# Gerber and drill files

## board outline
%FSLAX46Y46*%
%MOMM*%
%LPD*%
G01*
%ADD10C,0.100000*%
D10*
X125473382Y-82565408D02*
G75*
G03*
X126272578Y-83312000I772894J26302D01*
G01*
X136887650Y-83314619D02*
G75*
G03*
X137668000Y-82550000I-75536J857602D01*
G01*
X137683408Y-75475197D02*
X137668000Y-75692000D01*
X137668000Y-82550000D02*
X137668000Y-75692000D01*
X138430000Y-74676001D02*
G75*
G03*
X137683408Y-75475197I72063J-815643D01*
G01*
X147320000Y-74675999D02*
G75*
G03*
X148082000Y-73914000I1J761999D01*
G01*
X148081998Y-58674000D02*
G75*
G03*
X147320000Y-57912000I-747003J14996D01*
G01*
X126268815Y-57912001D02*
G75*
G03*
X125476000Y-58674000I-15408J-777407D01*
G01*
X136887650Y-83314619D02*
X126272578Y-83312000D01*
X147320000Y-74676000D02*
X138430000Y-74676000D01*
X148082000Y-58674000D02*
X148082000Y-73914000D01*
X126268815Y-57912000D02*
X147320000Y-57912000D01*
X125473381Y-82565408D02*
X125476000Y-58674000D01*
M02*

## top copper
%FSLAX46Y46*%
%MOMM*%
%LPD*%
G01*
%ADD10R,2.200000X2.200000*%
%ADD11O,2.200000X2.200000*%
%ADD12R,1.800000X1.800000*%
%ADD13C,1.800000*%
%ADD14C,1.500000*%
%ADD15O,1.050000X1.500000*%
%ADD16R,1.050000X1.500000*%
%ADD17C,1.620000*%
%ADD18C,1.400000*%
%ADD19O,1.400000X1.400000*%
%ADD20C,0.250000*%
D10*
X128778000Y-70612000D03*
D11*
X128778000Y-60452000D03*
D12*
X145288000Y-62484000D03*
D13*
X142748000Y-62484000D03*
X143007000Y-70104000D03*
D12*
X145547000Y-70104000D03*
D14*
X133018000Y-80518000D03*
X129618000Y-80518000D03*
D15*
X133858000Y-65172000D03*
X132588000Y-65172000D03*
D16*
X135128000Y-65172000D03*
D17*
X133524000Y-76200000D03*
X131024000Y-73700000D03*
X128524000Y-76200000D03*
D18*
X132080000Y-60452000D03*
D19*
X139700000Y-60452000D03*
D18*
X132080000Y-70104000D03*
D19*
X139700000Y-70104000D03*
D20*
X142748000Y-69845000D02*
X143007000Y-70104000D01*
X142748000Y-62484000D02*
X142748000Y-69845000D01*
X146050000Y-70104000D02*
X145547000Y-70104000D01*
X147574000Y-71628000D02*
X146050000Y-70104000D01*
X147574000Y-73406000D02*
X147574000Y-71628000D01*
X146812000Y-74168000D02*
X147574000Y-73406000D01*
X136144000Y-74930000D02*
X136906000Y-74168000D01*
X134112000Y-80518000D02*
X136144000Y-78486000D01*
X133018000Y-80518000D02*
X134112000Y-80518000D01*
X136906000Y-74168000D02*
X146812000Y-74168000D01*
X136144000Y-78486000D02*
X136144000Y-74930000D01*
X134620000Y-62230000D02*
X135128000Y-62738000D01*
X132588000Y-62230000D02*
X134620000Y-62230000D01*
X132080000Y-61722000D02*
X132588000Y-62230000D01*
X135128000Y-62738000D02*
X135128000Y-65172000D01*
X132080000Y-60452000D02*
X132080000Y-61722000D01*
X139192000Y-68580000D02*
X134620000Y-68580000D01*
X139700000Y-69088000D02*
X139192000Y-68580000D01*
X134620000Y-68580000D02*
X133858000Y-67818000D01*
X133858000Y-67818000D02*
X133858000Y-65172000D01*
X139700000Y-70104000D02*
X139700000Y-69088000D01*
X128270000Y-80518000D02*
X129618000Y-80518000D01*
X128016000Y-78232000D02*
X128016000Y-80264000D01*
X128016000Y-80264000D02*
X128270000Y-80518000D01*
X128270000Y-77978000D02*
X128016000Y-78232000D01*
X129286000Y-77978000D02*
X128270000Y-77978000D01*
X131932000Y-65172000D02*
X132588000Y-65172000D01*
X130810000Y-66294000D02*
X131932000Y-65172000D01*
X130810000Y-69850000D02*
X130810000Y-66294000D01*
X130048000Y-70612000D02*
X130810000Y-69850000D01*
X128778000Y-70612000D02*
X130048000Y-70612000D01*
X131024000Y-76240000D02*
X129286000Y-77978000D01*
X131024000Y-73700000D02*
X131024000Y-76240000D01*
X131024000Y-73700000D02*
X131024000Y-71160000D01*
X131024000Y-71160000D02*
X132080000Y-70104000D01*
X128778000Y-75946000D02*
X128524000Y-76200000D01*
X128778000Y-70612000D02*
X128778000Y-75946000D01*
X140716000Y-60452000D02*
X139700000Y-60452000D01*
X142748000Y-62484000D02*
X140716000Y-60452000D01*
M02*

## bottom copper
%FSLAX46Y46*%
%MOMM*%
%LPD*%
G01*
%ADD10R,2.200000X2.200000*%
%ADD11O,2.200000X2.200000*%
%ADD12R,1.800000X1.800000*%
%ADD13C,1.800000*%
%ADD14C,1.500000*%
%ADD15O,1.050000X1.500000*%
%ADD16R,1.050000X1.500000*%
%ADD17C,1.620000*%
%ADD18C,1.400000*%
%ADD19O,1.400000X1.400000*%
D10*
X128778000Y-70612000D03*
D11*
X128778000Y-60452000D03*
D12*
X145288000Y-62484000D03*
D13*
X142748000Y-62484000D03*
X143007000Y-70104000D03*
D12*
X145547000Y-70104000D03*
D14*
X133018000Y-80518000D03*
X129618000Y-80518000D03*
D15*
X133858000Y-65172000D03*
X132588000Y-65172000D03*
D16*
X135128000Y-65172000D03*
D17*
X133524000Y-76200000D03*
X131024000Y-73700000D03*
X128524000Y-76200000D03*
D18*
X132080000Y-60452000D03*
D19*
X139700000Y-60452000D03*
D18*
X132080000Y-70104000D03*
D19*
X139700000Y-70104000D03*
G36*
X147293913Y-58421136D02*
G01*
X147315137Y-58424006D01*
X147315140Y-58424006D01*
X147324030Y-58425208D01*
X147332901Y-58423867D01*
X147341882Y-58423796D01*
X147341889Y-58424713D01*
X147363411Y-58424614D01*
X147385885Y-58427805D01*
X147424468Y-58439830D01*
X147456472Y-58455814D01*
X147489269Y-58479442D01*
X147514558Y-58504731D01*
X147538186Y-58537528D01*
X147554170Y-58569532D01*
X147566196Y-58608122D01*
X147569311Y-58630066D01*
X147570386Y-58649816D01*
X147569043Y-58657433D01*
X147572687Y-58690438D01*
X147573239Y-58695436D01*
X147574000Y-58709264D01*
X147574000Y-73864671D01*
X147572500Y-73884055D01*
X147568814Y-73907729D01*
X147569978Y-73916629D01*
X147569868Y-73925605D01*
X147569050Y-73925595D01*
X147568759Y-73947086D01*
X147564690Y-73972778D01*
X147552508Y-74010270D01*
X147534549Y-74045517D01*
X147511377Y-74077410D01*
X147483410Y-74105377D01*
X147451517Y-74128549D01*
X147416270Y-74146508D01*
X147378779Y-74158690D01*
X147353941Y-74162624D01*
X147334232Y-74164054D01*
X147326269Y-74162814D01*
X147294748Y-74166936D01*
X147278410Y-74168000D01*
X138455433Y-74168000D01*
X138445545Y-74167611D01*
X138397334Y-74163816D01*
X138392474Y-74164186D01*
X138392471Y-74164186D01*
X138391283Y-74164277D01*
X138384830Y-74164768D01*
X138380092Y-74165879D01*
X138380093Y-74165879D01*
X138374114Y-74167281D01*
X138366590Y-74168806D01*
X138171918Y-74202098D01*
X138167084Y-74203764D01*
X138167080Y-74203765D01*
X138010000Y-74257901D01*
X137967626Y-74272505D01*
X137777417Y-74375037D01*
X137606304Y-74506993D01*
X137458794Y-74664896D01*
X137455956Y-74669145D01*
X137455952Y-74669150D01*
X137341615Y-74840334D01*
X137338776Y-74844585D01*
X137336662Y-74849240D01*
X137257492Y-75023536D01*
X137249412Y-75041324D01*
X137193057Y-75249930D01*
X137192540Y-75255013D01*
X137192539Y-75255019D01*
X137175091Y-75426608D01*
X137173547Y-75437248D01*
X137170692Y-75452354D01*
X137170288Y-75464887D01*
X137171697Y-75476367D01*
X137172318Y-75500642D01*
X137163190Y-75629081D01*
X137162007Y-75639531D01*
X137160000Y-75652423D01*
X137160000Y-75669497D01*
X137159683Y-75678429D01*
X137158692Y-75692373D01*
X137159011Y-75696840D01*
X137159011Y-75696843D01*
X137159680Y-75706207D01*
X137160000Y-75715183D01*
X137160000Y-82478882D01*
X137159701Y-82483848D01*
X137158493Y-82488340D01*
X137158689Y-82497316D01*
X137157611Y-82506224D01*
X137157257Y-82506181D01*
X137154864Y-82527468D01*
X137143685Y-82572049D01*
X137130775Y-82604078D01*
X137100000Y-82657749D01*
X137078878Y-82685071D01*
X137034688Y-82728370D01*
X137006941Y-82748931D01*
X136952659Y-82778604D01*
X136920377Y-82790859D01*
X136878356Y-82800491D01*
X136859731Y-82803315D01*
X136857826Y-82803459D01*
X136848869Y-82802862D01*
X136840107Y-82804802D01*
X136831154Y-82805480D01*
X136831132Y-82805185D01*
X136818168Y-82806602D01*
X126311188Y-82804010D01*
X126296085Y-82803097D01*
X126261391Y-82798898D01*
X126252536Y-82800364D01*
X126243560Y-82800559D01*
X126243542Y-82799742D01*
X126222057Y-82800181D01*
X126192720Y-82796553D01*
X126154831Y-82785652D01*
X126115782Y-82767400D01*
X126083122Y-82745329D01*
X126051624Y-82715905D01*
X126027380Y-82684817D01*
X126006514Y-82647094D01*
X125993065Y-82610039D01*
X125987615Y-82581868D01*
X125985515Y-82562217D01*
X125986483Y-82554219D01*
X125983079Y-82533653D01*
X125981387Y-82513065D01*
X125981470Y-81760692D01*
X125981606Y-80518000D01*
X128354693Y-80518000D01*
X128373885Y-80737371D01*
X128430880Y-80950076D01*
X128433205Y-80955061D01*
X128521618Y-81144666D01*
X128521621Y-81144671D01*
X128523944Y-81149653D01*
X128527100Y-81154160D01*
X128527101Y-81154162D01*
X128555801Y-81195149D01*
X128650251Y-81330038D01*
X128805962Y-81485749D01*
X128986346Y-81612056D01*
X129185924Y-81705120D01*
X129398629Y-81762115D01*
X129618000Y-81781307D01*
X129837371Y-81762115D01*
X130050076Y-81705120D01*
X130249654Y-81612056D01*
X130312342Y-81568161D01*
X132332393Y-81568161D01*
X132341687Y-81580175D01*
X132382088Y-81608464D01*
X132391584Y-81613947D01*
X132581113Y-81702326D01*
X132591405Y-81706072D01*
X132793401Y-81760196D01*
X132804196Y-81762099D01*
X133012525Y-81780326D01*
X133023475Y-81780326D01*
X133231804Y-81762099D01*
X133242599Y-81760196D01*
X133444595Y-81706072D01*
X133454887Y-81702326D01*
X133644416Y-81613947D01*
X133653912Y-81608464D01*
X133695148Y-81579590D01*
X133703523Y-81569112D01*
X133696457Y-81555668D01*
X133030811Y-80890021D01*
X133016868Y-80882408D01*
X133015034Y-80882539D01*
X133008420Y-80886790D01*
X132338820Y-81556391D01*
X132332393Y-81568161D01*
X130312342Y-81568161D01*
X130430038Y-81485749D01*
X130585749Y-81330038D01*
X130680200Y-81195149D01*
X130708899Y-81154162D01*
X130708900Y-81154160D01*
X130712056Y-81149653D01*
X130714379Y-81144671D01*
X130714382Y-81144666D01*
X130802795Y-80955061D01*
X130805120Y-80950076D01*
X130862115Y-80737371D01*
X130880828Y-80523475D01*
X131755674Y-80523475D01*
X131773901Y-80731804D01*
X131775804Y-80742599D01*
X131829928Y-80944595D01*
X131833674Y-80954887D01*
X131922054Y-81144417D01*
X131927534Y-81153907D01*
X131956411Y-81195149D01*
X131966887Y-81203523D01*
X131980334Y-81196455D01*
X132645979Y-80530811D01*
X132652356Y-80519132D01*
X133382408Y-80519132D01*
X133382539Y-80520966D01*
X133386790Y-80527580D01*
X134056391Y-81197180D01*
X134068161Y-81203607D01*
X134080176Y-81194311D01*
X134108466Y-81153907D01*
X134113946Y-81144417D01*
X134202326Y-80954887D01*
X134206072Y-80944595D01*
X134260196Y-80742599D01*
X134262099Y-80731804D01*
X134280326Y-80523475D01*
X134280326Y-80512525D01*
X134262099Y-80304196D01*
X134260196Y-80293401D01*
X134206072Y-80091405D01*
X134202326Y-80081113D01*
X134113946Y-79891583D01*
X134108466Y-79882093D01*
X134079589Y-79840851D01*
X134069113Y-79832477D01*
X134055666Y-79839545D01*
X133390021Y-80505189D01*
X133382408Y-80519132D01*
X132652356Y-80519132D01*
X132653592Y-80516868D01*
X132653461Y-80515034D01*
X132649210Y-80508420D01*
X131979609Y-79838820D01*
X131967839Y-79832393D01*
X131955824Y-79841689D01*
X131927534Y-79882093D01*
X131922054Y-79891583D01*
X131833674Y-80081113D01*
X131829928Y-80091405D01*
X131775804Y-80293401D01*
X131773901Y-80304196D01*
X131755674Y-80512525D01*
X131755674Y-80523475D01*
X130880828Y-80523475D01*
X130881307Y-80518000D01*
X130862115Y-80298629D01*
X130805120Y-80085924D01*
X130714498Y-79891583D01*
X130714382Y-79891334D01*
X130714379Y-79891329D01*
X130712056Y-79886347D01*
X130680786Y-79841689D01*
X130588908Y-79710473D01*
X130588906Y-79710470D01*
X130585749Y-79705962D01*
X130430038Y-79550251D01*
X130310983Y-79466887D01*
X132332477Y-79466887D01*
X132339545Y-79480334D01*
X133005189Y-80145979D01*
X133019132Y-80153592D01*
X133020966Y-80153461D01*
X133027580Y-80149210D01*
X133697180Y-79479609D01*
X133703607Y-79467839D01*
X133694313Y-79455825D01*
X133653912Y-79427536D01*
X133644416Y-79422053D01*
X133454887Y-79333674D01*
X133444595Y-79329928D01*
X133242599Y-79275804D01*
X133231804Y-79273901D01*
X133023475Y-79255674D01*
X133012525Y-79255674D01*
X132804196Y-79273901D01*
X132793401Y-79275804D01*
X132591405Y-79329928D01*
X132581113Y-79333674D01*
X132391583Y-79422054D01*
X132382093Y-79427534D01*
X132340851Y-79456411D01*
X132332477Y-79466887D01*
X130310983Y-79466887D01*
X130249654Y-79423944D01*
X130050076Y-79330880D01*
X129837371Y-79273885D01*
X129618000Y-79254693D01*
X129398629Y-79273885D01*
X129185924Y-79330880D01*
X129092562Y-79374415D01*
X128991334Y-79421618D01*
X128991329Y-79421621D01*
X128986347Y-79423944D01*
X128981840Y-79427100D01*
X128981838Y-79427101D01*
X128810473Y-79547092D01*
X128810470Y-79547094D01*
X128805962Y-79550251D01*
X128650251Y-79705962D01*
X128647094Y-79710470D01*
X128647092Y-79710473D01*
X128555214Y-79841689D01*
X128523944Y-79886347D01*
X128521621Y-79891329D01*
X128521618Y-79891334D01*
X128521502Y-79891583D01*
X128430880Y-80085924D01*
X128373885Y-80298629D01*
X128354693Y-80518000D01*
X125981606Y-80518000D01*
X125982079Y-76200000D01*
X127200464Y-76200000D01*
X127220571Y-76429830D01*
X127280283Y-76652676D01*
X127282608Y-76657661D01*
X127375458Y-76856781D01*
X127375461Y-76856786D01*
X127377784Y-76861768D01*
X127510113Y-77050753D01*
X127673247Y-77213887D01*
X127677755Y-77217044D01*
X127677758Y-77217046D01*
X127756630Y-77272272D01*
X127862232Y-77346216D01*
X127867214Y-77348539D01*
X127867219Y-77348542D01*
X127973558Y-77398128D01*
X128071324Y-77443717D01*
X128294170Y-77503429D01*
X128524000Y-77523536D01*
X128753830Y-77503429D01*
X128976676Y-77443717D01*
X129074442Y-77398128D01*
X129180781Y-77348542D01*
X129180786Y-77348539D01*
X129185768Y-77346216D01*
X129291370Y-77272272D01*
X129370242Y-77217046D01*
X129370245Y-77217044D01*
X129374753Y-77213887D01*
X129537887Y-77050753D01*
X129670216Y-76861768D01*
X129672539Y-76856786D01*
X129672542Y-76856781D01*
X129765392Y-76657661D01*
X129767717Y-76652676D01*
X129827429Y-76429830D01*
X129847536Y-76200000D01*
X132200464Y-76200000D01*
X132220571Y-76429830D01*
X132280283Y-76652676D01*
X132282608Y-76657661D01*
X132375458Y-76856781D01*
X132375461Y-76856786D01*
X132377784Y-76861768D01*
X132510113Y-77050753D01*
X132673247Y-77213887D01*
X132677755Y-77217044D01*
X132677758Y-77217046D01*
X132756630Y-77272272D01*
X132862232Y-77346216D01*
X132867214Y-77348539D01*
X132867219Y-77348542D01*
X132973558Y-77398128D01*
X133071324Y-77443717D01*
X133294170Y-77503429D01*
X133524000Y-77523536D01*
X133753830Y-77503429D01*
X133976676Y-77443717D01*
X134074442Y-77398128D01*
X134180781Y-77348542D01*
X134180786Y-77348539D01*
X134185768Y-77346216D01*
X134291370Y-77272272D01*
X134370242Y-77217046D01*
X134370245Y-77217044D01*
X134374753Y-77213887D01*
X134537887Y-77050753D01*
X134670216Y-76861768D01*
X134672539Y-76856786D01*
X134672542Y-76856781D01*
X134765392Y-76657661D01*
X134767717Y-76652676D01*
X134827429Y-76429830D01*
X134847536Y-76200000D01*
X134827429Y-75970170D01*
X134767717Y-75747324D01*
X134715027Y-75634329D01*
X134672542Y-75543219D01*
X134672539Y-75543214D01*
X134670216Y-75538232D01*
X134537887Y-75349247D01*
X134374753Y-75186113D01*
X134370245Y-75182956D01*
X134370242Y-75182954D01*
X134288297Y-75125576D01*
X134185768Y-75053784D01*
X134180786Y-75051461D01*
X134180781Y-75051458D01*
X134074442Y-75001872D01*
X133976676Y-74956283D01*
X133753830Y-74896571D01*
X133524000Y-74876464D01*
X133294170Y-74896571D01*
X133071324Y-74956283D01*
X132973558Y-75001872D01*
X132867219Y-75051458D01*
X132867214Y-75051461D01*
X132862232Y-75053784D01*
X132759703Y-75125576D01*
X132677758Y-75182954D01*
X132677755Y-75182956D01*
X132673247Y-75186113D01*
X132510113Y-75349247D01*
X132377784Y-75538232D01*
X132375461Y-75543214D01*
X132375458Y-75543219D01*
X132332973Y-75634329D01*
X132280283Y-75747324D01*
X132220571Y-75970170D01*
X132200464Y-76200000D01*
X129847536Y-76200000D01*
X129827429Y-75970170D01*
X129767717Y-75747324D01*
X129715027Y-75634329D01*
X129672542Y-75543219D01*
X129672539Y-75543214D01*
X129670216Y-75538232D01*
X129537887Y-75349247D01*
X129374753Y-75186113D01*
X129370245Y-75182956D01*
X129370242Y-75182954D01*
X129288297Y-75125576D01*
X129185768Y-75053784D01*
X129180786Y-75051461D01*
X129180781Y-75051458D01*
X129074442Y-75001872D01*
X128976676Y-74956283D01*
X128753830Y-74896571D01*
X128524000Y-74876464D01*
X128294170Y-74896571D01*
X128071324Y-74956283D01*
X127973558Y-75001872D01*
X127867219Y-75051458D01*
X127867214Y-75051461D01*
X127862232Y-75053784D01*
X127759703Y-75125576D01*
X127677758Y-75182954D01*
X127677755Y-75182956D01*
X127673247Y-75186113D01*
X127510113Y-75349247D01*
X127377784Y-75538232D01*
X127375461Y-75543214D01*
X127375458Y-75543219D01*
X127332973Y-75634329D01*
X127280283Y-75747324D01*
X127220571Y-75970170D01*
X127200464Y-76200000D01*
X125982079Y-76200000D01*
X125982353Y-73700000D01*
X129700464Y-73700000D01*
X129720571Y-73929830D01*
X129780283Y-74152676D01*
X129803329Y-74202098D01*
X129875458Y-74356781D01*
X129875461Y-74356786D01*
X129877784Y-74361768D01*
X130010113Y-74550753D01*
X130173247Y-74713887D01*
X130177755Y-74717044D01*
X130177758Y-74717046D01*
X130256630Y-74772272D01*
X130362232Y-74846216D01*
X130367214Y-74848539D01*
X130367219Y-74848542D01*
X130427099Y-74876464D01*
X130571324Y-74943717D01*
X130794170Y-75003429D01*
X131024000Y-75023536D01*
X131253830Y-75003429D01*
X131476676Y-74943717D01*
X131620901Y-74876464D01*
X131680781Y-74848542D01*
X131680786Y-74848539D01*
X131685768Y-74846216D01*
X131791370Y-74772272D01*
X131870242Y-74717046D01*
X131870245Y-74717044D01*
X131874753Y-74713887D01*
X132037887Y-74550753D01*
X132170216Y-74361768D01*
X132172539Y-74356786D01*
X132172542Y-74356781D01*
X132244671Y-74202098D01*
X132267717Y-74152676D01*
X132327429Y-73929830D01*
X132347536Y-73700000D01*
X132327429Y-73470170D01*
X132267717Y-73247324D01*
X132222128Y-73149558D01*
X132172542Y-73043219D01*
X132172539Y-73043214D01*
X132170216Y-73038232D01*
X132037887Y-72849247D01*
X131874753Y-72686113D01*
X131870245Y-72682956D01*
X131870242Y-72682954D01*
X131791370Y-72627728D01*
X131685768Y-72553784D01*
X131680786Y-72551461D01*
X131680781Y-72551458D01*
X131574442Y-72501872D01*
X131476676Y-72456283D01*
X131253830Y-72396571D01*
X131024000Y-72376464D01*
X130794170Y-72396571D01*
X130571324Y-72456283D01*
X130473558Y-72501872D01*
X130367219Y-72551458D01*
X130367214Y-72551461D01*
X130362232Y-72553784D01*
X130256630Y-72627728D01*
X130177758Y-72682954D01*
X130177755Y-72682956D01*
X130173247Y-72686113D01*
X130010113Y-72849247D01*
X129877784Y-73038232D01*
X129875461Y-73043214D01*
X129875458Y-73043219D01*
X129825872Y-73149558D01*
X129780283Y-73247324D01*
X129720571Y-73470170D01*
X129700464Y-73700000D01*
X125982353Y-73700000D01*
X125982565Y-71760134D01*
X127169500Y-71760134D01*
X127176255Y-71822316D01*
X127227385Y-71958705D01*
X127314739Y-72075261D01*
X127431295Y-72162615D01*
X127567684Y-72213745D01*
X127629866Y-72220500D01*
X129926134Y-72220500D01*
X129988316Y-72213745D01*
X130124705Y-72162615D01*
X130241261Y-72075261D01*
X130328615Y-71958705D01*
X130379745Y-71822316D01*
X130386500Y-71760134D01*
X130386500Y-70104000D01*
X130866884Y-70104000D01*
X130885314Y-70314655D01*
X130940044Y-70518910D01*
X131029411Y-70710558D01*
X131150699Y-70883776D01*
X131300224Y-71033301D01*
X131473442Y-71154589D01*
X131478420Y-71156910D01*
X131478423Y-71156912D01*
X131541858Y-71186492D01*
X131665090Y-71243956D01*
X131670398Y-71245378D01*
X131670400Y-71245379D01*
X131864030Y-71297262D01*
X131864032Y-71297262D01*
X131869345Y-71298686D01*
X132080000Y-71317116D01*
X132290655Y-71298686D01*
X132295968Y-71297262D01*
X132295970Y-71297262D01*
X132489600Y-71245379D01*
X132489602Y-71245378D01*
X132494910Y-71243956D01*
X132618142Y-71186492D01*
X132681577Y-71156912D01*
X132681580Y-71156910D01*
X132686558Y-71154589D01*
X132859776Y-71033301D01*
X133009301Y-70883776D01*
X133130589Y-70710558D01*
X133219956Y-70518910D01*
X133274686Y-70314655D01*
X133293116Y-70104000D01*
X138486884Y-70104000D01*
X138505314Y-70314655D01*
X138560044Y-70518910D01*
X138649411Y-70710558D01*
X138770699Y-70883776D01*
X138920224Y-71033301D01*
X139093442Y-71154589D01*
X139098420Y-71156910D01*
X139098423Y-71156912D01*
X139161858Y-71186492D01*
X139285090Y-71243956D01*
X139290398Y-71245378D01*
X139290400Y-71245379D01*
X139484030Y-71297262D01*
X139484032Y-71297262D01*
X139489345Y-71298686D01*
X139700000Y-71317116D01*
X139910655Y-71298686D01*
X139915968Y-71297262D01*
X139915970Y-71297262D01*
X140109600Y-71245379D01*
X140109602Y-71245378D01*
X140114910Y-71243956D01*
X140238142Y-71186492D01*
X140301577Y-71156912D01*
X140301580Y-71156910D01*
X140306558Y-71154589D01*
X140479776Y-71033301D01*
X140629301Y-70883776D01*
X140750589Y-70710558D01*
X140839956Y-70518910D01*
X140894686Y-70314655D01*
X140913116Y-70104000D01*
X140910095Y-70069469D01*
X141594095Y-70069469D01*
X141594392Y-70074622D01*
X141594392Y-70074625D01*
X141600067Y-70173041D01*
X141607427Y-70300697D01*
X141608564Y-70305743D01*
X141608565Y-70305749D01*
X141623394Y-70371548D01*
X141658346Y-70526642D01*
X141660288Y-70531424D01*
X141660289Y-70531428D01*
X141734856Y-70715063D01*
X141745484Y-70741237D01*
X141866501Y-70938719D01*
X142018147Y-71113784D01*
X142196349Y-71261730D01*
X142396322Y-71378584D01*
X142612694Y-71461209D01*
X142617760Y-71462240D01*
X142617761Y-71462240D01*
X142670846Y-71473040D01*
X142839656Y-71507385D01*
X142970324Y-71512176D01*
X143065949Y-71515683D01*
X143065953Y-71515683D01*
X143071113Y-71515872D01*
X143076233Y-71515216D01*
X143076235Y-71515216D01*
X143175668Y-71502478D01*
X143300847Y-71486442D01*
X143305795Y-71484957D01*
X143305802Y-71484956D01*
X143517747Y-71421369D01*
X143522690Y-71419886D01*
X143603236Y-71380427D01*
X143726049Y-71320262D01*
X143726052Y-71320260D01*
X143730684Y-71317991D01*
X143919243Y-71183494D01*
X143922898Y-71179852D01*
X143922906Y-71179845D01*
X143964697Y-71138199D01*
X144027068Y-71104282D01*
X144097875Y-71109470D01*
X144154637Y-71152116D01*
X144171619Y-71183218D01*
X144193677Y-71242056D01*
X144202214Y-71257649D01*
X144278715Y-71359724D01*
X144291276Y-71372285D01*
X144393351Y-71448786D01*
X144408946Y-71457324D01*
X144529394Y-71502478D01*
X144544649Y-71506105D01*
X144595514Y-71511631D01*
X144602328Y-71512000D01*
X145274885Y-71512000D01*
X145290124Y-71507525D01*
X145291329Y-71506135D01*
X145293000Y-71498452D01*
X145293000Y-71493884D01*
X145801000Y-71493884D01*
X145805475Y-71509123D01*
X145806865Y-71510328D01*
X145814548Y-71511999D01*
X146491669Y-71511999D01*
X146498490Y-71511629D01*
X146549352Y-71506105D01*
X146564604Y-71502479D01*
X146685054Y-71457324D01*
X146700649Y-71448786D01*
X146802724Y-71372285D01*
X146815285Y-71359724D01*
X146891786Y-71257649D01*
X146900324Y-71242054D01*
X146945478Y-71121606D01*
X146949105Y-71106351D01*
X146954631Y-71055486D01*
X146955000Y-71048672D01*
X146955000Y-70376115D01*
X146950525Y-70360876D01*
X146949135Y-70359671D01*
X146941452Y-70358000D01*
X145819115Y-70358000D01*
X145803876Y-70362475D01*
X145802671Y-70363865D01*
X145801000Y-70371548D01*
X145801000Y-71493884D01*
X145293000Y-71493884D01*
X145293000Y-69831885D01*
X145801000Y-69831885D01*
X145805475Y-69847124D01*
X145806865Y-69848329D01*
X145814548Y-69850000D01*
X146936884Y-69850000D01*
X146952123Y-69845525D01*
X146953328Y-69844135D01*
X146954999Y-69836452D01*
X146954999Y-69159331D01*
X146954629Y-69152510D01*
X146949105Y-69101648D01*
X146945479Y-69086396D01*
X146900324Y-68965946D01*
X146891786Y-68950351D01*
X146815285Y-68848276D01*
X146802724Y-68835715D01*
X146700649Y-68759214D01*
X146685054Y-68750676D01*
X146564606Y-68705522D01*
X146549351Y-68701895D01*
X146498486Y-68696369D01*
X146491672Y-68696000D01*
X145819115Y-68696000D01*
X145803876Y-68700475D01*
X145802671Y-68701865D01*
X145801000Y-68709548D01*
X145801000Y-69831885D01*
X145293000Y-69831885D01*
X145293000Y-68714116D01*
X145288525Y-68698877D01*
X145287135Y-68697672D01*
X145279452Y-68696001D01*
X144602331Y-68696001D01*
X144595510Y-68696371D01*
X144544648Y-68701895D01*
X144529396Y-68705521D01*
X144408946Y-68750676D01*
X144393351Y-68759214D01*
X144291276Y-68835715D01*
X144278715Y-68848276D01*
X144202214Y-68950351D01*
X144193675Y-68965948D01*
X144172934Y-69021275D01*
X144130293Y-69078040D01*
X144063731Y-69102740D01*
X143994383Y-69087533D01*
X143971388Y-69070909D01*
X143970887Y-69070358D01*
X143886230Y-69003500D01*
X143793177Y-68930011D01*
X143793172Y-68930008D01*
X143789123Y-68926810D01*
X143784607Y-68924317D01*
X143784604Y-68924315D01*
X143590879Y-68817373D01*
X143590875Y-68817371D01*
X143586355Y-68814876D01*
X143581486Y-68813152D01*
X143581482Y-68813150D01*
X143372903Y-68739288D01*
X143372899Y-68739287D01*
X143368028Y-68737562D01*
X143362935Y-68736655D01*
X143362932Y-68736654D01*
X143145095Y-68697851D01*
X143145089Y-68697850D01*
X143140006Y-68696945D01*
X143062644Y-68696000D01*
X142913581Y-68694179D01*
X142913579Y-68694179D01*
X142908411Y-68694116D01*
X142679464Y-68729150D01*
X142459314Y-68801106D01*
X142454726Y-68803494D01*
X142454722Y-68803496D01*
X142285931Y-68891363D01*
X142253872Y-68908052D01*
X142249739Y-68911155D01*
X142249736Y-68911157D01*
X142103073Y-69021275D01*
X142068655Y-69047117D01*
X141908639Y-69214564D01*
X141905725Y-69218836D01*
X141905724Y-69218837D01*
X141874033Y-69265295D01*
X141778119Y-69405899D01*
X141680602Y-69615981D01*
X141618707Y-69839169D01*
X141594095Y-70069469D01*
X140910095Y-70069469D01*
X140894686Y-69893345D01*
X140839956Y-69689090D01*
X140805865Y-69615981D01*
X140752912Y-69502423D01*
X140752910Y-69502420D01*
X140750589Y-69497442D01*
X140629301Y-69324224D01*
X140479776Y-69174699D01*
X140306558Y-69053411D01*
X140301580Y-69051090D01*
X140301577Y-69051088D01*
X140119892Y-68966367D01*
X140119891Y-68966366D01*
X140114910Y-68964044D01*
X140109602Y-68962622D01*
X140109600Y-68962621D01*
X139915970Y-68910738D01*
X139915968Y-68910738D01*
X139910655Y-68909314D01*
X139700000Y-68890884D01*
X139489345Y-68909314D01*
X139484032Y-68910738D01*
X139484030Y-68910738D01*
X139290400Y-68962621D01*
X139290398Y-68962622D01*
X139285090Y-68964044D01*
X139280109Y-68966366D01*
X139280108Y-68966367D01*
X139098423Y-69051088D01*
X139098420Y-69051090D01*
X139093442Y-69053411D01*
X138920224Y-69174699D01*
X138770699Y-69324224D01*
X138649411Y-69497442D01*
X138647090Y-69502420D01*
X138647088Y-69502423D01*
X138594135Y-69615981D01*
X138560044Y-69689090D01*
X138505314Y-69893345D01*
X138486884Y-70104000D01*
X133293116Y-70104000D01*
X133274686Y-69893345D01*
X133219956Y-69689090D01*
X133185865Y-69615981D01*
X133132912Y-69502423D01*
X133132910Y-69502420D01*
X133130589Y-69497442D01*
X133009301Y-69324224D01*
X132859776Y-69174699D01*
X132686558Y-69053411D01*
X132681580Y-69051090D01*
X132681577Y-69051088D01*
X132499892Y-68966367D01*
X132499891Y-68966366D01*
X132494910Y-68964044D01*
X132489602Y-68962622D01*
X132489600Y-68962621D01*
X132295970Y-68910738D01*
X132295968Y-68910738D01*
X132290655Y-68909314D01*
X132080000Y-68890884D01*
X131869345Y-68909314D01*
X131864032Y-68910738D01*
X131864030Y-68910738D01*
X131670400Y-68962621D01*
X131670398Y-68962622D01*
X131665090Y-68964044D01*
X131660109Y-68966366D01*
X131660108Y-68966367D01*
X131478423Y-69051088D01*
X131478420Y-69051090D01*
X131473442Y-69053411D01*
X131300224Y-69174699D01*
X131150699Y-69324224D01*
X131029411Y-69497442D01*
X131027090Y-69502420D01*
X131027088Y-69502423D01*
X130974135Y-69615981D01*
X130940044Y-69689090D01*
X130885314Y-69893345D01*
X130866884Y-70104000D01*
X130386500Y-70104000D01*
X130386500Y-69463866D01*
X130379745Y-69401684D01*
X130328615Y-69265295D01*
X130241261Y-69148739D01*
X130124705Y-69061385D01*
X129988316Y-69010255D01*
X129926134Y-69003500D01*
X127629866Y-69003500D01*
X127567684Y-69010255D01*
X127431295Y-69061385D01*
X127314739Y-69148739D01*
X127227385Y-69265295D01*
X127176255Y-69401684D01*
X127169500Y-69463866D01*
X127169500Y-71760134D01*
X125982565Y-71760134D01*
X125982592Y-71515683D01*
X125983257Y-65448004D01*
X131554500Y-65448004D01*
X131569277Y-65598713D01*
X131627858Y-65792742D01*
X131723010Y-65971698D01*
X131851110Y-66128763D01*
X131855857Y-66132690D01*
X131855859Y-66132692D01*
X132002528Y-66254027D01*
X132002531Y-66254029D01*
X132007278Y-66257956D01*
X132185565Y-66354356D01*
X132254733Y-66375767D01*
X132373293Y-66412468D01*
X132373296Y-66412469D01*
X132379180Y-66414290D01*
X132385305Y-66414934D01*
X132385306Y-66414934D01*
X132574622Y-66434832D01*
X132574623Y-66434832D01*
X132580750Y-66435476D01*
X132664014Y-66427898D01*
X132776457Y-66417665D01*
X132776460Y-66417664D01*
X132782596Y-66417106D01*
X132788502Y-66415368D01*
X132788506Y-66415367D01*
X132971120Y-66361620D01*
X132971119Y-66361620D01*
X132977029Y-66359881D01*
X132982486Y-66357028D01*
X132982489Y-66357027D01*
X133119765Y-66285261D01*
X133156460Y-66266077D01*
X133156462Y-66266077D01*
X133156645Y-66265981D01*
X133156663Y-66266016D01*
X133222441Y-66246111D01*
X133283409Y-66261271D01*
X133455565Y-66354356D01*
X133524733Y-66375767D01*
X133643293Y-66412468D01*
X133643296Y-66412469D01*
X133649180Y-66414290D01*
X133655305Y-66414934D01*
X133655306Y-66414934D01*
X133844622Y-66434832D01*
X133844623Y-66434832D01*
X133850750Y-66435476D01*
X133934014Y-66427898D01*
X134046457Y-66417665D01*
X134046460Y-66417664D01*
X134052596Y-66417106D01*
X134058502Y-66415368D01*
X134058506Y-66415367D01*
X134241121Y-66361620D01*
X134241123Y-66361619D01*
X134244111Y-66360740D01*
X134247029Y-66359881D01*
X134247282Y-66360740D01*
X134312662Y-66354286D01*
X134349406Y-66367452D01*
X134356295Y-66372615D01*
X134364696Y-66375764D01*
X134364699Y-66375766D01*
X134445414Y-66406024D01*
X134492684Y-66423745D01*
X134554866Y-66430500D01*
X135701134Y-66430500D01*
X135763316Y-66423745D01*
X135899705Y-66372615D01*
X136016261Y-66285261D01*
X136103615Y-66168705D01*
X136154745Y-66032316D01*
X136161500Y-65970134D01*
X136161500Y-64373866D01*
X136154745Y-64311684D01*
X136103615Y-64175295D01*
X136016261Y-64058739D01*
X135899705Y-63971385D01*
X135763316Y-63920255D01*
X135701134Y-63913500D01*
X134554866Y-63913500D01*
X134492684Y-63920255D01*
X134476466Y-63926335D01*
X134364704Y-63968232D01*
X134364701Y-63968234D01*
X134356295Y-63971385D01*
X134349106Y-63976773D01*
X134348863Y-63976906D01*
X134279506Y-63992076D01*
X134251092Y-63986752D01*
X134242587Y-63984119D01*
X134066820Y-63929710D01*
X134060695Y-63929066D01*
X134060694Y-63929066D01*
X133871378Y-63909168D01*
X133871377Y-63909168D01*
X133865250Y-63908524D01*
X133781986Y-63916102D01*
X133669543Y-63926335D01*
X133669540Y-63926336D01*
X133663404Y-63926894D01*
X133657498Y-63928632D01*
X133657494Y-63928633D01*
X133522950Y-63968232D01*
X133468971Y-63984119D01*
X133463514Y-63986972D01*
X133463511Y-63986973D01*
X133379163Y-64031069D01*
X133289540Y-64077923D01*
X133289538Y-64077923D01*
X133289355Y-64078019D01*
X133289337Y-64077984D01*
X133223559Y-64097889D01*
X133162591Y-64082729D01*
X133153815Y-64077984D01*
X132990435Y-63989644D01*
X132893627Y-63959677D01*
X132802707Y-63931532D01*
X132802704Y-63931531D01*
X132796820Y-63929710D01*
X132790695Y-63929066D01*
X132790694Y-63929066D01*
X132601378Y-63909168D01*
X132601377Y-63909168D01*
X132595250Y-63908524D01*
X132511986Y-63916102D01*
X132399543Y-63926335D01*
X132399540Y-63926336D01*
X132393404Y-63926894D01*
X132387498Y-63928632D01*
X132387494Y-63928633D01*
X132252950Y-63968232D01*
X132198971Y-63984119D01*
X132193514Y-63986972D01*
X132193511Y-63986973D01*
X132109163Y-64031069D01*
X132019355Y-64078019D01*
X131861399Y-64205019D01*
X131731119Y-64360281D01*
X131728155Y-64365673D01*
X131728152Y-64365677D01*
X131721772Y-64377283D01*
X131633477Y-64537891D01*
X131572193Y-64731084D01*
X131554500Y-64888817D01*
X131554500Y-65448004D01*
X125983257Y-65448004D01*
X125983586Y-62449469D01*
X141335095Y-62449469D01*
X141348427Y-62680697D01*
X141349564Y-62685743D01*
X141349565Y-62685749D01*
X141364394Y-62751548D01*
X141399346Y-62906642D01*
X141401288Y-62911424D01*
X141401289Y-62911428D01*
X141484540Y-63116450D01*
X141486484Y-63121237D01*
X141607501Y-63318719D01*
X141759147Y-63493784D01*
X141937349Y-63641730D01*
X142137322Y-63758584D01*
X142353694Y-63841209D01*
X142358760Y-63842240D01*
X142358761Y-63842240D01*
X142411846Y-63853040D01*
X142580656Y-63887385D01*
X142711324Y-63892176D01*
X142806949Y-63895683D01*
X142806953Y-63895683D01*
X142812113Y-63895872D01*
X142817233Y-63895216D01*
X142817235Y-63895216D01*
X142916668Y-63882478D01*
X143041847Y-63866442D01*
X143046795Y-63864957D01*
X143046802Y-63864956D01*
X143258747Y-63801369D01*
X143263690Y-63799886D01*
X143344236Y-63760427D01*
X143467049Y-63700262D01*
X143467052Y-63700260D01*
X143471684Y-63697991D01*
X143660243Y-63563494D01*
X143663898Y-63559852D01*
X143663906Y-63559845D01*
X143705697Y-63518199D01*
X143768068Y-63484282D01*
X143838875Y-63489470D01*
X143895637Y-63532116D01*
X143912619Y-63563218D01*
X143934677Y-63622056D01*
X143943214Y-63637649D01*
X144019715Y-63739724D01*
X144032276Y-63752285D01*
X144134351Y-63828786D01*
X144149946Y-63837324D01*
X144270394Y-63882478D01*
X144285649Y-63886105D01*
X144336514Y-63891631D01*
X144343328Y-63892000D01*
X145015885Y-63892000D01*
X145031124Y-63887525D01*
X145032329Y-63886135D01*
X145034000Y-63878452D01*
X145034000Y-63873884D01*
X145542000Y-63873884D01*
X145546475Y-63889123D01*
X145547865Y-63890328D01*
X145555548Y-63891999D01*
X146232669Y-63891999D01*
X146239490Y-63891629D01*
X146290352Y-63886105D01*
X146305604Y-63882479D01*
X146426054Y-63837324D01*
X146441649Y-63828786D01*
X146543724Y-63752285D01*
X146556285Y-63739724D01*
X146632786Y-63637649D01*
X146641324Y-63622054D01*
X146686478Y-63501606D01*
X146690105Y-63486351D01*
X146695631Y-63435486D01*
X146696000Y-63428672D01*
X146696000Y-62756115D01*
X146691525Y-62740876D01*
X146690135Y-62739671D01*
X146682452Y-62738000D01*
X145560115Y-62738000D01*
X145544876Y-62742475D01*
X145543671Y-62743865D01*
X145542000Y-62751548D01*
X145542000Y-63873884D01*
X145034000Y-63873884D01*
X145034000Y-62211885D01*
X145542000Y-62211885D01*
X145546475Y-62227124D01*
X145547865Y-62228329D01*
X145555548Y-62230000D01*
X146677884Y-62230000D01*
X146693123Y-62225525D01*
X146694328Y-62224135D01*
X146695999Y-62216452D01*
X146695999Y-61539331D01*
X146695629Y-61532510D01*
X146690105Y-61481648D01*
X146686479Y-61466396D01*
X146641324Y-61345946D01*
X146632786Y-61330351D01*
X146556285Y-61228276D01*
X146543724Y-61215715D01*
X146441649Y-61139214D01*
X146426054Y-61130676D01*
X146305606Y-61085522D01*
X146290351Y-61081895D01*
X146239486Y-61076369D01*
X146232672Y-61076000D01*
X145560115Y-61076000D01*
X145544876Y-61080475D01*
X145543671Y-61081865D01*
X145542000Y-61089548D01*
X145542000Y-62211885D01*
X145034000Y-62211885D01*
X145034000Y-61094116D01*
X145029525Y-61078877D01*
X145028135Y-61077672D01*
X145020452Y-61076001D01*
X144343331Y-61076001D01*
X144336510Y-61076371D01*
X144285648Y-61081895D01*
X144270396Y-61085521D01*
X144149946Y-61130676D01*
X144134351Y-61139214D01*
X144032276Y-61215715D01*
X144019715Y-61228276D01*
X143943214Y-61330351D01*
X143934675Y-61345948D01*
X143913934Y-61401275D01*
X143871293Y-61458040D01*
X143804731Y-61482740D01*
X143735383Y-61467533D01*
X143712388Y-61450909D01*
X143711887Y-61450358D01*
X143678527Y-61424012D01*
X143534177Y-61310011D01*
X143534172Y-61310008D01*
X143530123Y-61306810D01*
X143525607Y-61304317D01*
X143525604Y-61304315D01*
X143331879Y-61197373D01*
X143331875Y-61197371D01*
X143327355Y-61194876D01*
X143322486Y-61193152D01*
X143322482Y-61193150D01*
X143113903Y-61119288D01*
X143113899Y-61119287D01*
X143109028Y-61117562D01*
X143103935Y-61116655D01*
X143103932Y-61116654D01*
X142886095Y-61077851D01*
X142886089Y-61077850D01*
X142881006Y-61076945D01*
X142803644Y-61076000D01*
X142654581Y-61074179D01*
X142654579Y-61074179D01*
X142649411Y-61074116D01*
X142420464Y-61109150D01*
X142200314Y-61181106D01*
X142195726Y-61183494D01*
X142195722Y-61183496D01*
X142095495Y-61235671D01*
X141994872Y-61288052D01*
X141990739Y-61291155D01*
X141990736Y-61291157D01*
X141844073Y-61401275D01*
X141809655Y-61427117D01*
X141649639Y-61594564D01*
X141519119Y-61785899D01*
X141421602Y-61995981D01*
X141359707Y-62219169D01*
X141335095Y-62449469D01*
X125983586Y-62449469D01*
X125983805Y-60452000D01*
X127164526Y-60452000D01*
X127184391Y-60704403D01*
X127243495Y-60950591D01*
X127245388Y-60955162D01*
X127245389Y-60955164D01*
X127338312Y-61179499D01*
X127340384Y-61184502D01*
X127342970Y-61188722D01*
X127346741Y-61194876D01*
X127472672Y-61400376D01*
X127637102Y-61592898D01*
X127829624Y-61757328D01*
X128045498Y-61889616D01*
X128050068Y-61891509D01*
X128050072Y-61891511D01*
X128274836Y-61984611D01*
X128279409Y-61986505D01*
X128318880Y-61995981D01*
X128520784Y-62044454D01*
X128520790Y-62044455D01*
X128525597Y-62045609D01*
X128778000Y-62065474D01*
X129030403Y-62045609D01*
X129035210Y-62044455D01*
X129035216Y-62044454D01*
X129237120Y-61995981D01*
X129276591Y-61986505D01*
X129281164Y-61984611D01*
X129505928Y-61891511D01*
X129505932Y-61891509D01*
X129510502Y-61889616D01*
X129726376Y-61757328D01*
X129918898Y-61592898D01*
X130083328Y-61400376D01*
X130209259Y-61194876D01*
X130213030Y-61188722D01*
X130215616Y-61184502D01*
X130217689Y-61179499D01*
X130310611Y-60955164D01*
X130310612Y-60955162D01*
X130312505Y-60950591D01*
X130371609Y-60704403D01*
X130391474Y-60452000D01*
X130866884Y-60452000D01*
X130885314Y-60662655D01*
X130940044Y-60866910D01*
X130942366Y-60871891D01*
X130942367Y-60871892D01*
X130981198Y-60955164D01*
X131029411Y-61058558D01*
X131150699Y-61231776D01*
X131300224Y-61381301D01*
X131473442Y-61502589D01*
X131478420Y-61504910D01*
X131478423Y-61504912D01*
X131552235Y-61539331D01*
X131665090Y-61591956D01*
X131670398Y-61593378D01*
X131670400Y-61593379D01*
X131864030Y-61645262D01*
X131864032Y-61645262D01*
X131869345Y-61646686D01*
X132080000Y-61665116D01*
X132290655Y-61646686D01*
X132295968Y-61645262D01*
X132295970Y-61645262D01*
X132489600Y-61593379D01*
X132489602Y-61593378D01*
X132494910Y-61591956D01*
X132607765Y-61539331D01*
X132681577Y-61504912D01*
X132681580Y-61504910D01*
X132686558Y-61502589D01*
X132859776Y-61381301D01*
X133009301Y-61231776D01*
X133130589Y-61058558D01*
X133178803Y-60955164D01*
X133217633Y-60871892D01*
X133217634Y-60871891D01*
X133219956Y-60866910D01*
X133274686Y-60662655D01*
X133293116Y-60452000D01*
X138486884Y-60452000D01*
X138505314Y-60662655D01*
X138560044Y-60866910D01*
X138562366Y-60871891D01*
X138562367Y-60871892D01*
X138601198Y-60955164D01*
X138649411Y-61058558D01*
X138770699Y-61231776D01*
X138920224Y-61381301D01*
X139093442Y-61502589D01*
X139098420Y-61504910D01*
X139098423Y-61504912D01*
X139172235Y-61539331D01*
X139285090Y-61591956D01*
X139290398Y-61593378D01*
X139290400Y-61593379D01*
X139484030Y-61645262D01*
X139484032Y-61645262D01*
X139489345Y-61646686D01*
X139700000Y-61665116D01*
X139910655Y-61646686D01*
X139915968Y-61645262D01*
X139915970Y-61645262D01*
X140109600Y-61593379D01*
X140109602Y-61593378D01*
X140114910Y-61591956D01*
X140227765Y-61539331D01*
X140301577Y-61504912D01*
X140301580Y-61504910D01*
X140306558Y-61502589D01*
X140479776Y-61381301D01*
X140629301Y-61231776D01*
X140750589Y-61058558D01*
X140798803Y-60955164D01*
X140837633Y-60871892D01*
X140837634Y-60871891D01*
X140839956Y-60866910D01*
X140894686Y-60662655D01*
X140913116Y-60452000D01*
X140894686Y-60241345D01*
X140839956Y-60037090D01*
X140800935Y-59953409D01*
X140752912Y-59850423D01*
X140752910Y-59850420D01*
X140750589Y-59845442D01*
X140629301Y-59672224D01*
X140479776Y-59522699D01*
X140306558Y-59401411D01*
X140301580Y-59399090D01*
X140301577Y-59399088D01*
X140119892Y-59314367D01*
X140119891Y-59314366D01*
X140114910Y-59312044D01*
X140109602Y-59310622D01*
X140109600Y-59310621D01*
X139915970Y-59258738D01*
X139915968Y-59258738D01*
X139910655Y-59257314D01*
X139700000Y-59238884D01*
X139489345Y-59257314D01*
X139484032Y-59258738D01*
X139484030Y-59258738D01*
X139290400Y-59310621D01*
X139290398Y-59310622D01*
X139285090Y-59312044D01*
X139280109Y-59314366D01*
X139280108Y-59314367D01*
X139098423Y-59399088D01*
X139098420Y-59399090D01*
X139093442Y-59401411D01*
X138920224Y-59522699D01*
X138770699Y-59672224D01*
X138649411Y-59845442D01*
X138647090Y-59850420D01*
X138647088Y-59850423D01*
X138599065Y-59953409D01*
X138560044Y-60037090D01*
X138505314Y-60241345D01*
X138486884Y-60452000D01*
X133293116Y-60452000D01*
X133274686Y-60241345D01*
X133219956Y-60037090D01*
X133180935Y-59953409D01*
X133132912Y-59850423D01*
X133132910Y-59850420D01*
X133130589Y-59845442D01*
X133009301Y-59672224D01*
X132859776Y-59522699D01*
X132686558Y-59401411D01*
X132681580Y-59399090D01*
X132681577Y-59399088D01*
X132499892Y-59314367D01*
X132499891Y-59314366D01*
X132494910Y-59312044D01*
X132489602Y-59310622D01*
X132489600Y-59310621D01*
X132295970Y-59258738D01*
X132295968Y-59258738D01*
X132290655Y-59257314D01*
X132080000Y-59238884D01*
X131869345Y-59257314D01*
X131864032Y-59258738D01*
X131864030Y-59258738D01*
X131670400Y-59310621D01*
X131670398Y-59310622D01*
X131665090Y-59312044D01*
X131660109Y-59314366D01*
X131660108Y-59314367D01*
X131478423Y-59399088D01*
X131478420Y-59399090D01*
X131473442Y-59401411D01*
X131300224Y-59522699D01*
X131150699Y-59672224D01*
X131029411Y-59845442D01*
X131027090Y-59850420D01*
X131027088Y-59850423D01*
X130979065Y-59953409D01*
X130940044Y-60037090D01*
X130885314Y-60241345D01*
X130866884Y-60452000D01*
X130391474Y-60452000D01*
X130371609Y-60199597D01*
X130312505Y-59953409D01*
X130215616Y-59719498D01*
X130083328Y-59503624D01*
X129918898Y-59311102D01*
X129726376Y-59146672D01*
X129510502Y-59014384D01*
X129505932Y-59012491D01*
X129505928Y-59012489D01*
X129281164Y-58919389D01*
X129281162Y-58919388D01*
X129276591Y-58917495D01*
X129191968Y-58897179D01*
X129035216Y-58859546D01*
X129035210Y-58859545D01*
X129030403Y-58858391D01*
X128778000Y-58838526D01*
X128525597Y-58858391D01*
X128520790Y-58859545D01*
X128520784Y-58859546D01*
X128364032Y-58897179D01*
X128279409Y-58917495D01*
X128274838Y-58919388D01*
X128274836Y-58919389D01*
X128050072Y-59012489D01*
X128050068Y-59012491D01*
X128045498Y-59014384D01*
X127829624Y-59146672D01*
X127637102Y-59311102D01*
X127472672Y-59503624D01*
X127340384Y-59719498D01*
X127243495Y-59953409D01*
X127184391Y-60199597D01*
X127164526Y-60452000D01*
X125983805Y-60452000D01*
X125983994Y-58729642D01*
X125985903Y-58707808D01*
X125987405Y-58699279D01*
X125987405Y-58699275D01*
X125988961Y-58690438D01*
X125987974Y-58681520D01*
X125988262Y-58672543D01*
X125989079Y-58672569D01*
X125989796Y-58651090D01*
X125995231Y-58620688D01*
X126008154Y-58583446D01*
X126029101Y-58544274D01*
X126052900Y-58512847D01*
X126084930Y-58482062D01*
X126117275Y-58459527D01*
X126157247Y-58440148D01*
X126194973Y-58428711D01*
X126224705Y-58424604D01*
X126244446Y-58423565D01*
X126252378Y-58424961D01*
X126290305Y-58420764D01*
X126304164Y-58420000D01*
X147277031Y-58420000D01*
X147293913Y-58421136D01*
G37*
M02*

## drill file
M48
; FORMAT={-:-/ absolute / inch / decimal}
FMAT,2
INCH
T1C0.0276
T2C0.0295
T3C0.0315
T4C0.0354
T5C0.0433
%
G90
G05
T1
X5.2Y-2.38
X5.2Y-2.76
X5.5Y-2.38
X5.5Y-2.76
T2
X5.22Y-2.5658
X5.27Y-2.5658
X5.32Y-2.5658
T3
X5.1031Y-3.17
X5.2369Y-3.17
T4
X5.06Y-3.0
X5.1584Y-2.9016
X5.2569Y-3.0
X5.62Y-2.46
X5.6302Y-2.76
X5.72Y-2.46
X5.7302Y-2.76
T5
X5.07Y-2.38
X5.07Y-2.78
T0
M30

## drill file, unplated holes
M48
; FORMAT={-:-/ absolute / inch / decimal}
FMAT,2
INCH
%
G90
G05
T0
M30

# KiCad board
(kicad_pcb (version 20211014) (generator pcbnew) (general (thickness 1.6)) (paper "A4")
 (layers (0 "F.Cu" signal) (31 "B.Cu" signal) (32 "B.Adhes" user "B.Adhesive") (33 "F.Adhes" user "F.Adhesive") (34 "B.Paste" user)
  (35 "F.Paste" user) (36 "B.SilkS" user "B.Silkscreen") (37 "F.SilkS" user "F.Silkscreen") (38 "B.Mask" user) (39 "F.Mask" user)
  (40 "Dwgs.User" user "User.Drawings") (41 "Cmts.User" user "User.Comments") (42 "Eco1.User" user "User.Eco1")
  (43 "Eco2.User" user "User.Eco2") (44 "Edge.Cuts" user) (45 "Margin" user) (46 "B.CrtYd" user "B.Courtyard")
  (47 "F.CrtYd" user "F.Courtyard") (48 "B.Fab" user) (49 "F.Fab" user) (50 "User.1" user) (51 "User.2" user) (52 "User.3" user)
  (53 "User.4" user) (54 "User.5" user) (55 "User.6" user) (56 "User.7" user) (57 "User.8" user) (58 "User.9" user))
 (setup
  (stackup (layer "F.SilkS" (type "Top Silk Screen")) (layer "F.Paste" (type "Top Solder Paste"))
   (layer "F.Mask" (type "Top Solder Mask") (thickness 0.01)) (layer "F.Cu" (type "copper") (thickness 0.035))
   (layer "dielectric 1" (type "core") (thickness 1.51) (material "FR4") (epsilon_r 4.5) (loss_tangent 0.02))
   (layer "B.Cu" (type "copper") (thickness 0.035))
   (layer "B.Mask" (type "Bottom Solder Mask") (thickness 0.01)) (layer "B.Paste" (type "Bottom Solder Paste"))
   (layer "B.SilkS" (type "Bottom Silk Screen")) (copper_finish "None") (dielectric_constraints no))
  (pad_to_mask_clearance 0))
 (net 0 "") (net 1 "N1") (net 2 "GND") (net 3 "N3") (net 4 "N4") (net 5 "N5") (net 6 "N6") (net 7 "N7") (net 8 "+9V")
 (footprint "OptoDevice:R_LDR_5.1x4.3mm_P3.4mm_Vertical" (layer "F.Cu") (at 129.618 80.518)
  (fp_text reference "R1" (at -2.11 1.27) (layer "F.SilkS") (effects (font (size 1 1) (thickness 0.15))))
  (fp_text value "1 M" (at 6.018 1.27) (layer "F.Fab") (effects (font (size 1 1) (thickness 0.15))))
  (pad "1" thru_hole circle locked (at 0 0) (size 1.5 1.5) (drill 0.8) (layers *.Cu *.Mask) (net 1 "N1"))
  (pad "2" thru_hole circle locked (at 3.4 0) (size 1.5 1.5) (drill 0.8) (layers *.Cu *.Mask) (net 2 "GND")))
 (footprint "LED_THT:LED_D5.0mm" (layer "F.Cu") (at 145.288 62.484 180)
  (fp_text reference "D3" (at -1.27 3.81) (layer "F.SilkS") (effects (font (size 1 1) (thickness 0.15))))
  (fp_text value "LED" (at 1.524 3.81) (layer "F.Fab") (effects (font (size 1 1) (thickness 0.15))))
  (pad "1" thru_hole rect locked (at 0 0 180) (size 1.8 1.8) (drill 0.9) (layers *.Cu *.Mask) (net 2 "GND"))
  (pad "2" thru_hole circle locked (at 2.54 0 180) (size 1.8 1.8) (drill 0.9) (layers *.Cu *.Mask) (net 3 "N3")))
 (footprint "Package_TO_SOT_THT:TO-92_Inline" (layer "F.Cu") (at 135.128 65.172 180)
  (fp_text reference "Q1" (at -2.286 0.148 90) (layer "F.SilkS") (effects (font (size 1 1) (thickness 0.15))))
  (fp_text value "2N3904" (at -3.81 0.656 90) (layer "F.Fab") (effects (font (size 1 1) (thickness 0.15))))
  (pad "1" thru_hole rect locked (at 0 0 180) (size 1.05 1.5) (drill 0.75) (layers *.Cu *.Mask) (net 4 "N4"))
  (pad "2" thru_hole oval locked (at 1.27 0 180) (size 1.05 1.5) (drill 0.75) (layers *.Cu *.Mask) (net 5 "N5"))
  (pad "3" thru_hole oval locked (at 2.54 0 180) (size 1.05 1.5) (drill 0.75) (layers *.Cu *.Mask) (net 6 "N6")))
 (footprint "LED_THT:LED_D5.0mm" (layer "F.Cu") (at 145.547 70.104 180)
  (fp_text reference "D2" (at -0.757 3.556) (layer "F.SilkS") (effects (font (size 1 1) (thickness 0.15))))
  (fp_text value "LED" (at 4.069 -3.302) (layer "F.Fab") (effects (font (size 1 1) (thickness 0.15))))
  (pad "1" thru_hole rect locked (at 0 0 180) (size 1.8 1.8) (drill 0.9) (layers *.Cu *.Mask) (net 2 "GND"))
  (pad "2" thru_hole circle locked (at 2.54 0 180) (size 1.8 1.8) (drill 0.9) (layers *.Cu *.Mask) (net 3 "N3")))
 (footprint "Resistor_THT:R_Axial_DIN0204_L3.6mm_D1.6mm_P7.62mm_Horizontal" (layer "F.Cu") (at 132.08 70.104)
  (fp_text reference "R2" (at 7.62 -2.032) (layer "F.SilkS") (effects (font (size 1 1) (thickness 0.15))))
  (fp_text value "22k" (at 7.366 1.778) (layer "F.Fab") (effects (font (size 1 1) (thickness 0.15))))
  (pad "1" thru_hole circle locked (at 0 0) (size 1.4 1.4) (drill 0.7) (layers *.Cu *.Mask) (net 1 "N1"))
  (pad "2" thru_hole oval locked (at 7.62 0) (size 1.4 1.4) (drill 0.7) (layers *.Cu *.Mask) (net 5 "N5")))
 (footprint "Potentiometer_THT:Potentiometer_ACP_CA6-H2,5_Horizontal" (layer "F.Cu") (at 128.524 76.2 90)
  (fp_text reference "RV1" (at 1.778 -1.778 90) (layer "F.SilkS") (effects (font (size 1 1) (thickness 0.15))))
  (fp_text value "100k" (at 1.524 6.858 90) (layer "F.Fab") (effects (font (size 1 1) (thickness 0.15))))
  (pad "1" thru_hole circle locked (at 0 0 90) (size 1.62 1.62) (drill 0.9) (layers *.Cu *.Mask) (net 6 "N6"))
  (pad "2" thru_hole circle locked (at 2.5 2.5 90) (size 1.62 1.62) (drill 0.9) (layers *.Cu *.Mask) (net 1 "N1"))
  (pad "3" thru_hole circle locked (at 0 5 90) (size 1.62 1.62) (drill 0.9) (layers *.Cu *.Mask) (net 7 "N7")))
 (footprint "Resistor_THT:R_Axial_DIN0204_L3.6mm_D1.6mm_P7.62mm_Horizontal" (layer "F.Cu") (at 132.08 60.452)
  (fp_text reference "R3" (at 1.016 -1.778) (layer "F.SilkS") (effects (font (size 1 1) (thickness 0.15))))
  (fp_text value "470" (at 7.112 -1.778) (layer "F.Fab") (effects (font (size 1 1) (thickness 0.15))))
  (pad "1" thru_hole circle locked (at 0 0) (size 1.4 1.4) (drill 0.7) (layers *.Cu *.Mask) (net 4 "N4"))
  (pad "2" thru_hole oval locked (at 7.62 0) (size 1.4 1.4) (drill 0.7) (layers *.Cu *.Mask) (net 3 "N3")))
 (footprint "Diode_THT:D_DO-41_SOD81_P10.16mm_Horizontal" (layer "F.Cu") (at 128.778 70.612 90)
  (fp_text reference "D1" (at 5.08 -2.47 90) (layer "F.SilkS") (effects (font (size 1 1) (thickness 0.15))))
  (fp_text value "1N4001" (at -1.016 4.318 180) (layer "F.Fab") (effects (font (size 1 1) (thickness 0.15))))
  (pad "1" thru_hole rect locked (at 0 0 90) (size 2.2 2.2) (drill 1.1) (layers *.Cu *.Mask) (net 6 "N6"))
  (pad "2" thru_hole oval locked (at 10.16 0 90) (size 2.2 2.2) (drill 1.1) (layers *.Cu *.Mask) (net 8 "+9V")))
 (gr_line locked (start 137.668 82.55) (end 137.668 75.692) (layer "Edge.Cuts") (width 0.1))
 (gr_arc (start 137.683408 75.475197) (mid 137.903713 74.932678) (end 138.43 74.676) (layer "Edge.Cuts") (width 0.1))
 (gr_line locked (start 125.473381 82.565408) (end 125.476 58.674) (layer "Edge.Cuts") (width 0.1))
 (gr_line locked (start 147.32 74.676) (end 138.43 74.676) (layer "Edge.Cuts") (width 0.1))
 (gr_arc locked (start 148.082 73.914) (mid 147.858815 74.452815) (end 147.32 74.676) (layer "Edge.Cuts") (width 0.1))
 (gr_arc locked (start 126.272578 83.312) (mid 125.718356 83.104223) (end 125.473381 82.565408) (layer "Edge.Cuts") (width 0.1))
 (gr_arc (start 137.668 82.55) (mid 137.414648 83.071947) (end 136.88765 83.314619) (layer "Edge.Cuts") (width 0.1))
 (gr_arc locked (start 147.32 57.912) (mid 147.863313 58.130686) (end 148.082 58.674) (layer "Edge.Cuts") (width 0.1))
 (gr_line (start 137.683408 75.475197) (end 137.668 75.692) (layer "Edge.Cuts") (width 0.1))
 (gr_arc locked (start 125.476 58.674) (mid 125.714592 58.128803) (end 126.268815 57.912) (layer "Edge.Cuts") (width 0.1))
 (gr_line (start 136.88765 83.314619) (end 126.272578 83.312) (layer "Edge.Cuts") (width 0.1))
 (gr_line locked (start 148.082 58.674) (end 148.082 73.914) (layer "Edge.Cuts") (width 0.1))
 (gr_line (start 126.268815 57.912) (end 147.32 57.912) (layer "Edge.Cuts") (width 0.1))
 (segment (start 135.128 62.738) (end 135.128 65.172) (width 0.25) (layer "F.Cu") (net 4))
 (segment (start 132.08 60.452) (end 132.08 61.722) (width 0.25) (layer "F.Cu") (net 4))
 (segment (start 134.62 62.23) (end 135.128 62.738) (width 0.25) (layer "F.Cu") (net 4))
 (segment (start 132.08 61.722) (end 132.588 62.23) (width 0.25) (layer "F.Cu") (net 4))
 (segment (start 132.588 62.23) (end 134.62 62.23) (width 0.25) (layer "F.Cu") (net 4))
 (segment (start 131.024 71.16) (end 132.08 70.104) (width 0.25) (layer "F.Cu") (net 1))
 (segment (start 131.024 76.24) (end 129.286 77.978) (width 0.25) (layer "F.Cu") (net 1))
 (segment (start 128.27 77.978) (end 128.016 78.232) (width 0.25) (layer "F.Cu") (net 1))
 (segment (start 128.27 80.518) (end 129.618 80.518) (width 0.25) (layer "F.Cu") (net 1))
 (segment (start 128.016 78.232) (end 128.016 80.264) (width 0.25) (layer "F.Cu") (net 1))
 (segment (start 131.024 73.7) (end 131.024 76.24) (width 0.25) (layer "F.Cu") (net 1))
 (segment (start 129.286 77.978) (end 128.27 77.978) (width 0.25) (layer "F.Cu") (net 1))
 (segment (start 128.016 80.264) (end 128.27 80.518) (width 0.25) (layer "F.Cu") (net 1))
 (segment (start 131.024 73.7) (end 131.024 71.16) (width 0.25) (layer "F.Cu") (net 1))
 (segment (start 147.574 73.406) (end 147.574 71.628) (width 0.25) (layer "F.Cu") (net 2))
 (segment (start 146.812 74.168) (end 147.574 73.406) (width 0.25) (layer "F.Cu") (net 2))
 (segment (start 133.018 80.518) (end 134.112 80.518) (width 0.25) (layer "F.Cu") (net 2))
 (segment (start 146.05 70.104) (end 145.547 70.104) (width 0.25) (layer "F.Cu") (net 2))
 (segment (start 136.144 74.93) (end 136.906 74.168) (width 0.25) (layer "F.Cu") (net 2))
 (segment (start 136.906 74.168) (end 146.812 74.168) (width 0.25) (layer "F.Cu") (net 2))
 (segment (start 134.112 80.518) (end 136.144 78.486) (width 0.25) (layer "F.Cu") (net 2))
 (segment (start 147.574 71.628) (end 146.05 70.104) (width 0.25) (layer "F.Cu") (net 2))
 (segment (start 136.144 78.486) (end 136.144 74.93) (width 0.25) (layer "F.Cu") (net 2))
 (segment (start 128.778 70.612) (end 130.048 70.612) (width 0.25) (layer "F.Cu") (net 6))
 (segment (start 130.81 69.85) (end 130.81 66.294) (width 0.25) (layer "F.Cu") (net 6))
 (segment (start 128.778 75.946) (end 128.524 76.2) (width 0.25) (layer "F.Cu") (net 6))
 (segment (start 131.932 65.172) (end 132.588 65.172) (width 0.25) (layer "F.Cu") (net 6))
 (segment (start 130.81 66.294) (end 131.932 65.172) (width 0.25) (layer "F.Cu") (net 6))
 (segment (start 130.048 70.612) (end 130.81 69.85) (width 0.25) (layer "F.Cu") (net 6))
 (segment (start 128.778 70.612) (end 128.778 75.946) (width 0.25) (layer "F.Cu") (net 6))
 (segment (start 142.748 62.484) (end 142.748 69.845) (width 0.25) (layer "F.Cu") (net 3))
 (segment (start 142.748 69.845) (end 143.007 70.104) (width 0.25) (layer "F.Cu") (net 3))
 (segment (start 140.716 60.452) (end 139.7 60.452) (width 0.25) (layer "F.Cu") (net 3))
 (segment (start 142.748 62.484) (end 140.716 60.452) (width 0.25) (layer "F.Cu") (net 3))
 (segment (start 139.7 70.104) (end 139.7 69.088) (width 0.25) (layer "F.Cu") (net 5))
 (segment (start 133.858 67.818) (end 133.858 65.172) (width 0.25) (layer "F.Cu") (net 5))
 (segment (start 139.192 68.58) (end 134.62 68.58) (width 0.25) (layer "F.Cu") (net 5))
 (segment (start 139.7 69.088) (end 139.192 68.58) (width 0.25) (layer "F.Cu") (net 5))
 (segment (start 134.62 68.58) (end 133.858 67.818) (width 0.25) (layer "F.Cu") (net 5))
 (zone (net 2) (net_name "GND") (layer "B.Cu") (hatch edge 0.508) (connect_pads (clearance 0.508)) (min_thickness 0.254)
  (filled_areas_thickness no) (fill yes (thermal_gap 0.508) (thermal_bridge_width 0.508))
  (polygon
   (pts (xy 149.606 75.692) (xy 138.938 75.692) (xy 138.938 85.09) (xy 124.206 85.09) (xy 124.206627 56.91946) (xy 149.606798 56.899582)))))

